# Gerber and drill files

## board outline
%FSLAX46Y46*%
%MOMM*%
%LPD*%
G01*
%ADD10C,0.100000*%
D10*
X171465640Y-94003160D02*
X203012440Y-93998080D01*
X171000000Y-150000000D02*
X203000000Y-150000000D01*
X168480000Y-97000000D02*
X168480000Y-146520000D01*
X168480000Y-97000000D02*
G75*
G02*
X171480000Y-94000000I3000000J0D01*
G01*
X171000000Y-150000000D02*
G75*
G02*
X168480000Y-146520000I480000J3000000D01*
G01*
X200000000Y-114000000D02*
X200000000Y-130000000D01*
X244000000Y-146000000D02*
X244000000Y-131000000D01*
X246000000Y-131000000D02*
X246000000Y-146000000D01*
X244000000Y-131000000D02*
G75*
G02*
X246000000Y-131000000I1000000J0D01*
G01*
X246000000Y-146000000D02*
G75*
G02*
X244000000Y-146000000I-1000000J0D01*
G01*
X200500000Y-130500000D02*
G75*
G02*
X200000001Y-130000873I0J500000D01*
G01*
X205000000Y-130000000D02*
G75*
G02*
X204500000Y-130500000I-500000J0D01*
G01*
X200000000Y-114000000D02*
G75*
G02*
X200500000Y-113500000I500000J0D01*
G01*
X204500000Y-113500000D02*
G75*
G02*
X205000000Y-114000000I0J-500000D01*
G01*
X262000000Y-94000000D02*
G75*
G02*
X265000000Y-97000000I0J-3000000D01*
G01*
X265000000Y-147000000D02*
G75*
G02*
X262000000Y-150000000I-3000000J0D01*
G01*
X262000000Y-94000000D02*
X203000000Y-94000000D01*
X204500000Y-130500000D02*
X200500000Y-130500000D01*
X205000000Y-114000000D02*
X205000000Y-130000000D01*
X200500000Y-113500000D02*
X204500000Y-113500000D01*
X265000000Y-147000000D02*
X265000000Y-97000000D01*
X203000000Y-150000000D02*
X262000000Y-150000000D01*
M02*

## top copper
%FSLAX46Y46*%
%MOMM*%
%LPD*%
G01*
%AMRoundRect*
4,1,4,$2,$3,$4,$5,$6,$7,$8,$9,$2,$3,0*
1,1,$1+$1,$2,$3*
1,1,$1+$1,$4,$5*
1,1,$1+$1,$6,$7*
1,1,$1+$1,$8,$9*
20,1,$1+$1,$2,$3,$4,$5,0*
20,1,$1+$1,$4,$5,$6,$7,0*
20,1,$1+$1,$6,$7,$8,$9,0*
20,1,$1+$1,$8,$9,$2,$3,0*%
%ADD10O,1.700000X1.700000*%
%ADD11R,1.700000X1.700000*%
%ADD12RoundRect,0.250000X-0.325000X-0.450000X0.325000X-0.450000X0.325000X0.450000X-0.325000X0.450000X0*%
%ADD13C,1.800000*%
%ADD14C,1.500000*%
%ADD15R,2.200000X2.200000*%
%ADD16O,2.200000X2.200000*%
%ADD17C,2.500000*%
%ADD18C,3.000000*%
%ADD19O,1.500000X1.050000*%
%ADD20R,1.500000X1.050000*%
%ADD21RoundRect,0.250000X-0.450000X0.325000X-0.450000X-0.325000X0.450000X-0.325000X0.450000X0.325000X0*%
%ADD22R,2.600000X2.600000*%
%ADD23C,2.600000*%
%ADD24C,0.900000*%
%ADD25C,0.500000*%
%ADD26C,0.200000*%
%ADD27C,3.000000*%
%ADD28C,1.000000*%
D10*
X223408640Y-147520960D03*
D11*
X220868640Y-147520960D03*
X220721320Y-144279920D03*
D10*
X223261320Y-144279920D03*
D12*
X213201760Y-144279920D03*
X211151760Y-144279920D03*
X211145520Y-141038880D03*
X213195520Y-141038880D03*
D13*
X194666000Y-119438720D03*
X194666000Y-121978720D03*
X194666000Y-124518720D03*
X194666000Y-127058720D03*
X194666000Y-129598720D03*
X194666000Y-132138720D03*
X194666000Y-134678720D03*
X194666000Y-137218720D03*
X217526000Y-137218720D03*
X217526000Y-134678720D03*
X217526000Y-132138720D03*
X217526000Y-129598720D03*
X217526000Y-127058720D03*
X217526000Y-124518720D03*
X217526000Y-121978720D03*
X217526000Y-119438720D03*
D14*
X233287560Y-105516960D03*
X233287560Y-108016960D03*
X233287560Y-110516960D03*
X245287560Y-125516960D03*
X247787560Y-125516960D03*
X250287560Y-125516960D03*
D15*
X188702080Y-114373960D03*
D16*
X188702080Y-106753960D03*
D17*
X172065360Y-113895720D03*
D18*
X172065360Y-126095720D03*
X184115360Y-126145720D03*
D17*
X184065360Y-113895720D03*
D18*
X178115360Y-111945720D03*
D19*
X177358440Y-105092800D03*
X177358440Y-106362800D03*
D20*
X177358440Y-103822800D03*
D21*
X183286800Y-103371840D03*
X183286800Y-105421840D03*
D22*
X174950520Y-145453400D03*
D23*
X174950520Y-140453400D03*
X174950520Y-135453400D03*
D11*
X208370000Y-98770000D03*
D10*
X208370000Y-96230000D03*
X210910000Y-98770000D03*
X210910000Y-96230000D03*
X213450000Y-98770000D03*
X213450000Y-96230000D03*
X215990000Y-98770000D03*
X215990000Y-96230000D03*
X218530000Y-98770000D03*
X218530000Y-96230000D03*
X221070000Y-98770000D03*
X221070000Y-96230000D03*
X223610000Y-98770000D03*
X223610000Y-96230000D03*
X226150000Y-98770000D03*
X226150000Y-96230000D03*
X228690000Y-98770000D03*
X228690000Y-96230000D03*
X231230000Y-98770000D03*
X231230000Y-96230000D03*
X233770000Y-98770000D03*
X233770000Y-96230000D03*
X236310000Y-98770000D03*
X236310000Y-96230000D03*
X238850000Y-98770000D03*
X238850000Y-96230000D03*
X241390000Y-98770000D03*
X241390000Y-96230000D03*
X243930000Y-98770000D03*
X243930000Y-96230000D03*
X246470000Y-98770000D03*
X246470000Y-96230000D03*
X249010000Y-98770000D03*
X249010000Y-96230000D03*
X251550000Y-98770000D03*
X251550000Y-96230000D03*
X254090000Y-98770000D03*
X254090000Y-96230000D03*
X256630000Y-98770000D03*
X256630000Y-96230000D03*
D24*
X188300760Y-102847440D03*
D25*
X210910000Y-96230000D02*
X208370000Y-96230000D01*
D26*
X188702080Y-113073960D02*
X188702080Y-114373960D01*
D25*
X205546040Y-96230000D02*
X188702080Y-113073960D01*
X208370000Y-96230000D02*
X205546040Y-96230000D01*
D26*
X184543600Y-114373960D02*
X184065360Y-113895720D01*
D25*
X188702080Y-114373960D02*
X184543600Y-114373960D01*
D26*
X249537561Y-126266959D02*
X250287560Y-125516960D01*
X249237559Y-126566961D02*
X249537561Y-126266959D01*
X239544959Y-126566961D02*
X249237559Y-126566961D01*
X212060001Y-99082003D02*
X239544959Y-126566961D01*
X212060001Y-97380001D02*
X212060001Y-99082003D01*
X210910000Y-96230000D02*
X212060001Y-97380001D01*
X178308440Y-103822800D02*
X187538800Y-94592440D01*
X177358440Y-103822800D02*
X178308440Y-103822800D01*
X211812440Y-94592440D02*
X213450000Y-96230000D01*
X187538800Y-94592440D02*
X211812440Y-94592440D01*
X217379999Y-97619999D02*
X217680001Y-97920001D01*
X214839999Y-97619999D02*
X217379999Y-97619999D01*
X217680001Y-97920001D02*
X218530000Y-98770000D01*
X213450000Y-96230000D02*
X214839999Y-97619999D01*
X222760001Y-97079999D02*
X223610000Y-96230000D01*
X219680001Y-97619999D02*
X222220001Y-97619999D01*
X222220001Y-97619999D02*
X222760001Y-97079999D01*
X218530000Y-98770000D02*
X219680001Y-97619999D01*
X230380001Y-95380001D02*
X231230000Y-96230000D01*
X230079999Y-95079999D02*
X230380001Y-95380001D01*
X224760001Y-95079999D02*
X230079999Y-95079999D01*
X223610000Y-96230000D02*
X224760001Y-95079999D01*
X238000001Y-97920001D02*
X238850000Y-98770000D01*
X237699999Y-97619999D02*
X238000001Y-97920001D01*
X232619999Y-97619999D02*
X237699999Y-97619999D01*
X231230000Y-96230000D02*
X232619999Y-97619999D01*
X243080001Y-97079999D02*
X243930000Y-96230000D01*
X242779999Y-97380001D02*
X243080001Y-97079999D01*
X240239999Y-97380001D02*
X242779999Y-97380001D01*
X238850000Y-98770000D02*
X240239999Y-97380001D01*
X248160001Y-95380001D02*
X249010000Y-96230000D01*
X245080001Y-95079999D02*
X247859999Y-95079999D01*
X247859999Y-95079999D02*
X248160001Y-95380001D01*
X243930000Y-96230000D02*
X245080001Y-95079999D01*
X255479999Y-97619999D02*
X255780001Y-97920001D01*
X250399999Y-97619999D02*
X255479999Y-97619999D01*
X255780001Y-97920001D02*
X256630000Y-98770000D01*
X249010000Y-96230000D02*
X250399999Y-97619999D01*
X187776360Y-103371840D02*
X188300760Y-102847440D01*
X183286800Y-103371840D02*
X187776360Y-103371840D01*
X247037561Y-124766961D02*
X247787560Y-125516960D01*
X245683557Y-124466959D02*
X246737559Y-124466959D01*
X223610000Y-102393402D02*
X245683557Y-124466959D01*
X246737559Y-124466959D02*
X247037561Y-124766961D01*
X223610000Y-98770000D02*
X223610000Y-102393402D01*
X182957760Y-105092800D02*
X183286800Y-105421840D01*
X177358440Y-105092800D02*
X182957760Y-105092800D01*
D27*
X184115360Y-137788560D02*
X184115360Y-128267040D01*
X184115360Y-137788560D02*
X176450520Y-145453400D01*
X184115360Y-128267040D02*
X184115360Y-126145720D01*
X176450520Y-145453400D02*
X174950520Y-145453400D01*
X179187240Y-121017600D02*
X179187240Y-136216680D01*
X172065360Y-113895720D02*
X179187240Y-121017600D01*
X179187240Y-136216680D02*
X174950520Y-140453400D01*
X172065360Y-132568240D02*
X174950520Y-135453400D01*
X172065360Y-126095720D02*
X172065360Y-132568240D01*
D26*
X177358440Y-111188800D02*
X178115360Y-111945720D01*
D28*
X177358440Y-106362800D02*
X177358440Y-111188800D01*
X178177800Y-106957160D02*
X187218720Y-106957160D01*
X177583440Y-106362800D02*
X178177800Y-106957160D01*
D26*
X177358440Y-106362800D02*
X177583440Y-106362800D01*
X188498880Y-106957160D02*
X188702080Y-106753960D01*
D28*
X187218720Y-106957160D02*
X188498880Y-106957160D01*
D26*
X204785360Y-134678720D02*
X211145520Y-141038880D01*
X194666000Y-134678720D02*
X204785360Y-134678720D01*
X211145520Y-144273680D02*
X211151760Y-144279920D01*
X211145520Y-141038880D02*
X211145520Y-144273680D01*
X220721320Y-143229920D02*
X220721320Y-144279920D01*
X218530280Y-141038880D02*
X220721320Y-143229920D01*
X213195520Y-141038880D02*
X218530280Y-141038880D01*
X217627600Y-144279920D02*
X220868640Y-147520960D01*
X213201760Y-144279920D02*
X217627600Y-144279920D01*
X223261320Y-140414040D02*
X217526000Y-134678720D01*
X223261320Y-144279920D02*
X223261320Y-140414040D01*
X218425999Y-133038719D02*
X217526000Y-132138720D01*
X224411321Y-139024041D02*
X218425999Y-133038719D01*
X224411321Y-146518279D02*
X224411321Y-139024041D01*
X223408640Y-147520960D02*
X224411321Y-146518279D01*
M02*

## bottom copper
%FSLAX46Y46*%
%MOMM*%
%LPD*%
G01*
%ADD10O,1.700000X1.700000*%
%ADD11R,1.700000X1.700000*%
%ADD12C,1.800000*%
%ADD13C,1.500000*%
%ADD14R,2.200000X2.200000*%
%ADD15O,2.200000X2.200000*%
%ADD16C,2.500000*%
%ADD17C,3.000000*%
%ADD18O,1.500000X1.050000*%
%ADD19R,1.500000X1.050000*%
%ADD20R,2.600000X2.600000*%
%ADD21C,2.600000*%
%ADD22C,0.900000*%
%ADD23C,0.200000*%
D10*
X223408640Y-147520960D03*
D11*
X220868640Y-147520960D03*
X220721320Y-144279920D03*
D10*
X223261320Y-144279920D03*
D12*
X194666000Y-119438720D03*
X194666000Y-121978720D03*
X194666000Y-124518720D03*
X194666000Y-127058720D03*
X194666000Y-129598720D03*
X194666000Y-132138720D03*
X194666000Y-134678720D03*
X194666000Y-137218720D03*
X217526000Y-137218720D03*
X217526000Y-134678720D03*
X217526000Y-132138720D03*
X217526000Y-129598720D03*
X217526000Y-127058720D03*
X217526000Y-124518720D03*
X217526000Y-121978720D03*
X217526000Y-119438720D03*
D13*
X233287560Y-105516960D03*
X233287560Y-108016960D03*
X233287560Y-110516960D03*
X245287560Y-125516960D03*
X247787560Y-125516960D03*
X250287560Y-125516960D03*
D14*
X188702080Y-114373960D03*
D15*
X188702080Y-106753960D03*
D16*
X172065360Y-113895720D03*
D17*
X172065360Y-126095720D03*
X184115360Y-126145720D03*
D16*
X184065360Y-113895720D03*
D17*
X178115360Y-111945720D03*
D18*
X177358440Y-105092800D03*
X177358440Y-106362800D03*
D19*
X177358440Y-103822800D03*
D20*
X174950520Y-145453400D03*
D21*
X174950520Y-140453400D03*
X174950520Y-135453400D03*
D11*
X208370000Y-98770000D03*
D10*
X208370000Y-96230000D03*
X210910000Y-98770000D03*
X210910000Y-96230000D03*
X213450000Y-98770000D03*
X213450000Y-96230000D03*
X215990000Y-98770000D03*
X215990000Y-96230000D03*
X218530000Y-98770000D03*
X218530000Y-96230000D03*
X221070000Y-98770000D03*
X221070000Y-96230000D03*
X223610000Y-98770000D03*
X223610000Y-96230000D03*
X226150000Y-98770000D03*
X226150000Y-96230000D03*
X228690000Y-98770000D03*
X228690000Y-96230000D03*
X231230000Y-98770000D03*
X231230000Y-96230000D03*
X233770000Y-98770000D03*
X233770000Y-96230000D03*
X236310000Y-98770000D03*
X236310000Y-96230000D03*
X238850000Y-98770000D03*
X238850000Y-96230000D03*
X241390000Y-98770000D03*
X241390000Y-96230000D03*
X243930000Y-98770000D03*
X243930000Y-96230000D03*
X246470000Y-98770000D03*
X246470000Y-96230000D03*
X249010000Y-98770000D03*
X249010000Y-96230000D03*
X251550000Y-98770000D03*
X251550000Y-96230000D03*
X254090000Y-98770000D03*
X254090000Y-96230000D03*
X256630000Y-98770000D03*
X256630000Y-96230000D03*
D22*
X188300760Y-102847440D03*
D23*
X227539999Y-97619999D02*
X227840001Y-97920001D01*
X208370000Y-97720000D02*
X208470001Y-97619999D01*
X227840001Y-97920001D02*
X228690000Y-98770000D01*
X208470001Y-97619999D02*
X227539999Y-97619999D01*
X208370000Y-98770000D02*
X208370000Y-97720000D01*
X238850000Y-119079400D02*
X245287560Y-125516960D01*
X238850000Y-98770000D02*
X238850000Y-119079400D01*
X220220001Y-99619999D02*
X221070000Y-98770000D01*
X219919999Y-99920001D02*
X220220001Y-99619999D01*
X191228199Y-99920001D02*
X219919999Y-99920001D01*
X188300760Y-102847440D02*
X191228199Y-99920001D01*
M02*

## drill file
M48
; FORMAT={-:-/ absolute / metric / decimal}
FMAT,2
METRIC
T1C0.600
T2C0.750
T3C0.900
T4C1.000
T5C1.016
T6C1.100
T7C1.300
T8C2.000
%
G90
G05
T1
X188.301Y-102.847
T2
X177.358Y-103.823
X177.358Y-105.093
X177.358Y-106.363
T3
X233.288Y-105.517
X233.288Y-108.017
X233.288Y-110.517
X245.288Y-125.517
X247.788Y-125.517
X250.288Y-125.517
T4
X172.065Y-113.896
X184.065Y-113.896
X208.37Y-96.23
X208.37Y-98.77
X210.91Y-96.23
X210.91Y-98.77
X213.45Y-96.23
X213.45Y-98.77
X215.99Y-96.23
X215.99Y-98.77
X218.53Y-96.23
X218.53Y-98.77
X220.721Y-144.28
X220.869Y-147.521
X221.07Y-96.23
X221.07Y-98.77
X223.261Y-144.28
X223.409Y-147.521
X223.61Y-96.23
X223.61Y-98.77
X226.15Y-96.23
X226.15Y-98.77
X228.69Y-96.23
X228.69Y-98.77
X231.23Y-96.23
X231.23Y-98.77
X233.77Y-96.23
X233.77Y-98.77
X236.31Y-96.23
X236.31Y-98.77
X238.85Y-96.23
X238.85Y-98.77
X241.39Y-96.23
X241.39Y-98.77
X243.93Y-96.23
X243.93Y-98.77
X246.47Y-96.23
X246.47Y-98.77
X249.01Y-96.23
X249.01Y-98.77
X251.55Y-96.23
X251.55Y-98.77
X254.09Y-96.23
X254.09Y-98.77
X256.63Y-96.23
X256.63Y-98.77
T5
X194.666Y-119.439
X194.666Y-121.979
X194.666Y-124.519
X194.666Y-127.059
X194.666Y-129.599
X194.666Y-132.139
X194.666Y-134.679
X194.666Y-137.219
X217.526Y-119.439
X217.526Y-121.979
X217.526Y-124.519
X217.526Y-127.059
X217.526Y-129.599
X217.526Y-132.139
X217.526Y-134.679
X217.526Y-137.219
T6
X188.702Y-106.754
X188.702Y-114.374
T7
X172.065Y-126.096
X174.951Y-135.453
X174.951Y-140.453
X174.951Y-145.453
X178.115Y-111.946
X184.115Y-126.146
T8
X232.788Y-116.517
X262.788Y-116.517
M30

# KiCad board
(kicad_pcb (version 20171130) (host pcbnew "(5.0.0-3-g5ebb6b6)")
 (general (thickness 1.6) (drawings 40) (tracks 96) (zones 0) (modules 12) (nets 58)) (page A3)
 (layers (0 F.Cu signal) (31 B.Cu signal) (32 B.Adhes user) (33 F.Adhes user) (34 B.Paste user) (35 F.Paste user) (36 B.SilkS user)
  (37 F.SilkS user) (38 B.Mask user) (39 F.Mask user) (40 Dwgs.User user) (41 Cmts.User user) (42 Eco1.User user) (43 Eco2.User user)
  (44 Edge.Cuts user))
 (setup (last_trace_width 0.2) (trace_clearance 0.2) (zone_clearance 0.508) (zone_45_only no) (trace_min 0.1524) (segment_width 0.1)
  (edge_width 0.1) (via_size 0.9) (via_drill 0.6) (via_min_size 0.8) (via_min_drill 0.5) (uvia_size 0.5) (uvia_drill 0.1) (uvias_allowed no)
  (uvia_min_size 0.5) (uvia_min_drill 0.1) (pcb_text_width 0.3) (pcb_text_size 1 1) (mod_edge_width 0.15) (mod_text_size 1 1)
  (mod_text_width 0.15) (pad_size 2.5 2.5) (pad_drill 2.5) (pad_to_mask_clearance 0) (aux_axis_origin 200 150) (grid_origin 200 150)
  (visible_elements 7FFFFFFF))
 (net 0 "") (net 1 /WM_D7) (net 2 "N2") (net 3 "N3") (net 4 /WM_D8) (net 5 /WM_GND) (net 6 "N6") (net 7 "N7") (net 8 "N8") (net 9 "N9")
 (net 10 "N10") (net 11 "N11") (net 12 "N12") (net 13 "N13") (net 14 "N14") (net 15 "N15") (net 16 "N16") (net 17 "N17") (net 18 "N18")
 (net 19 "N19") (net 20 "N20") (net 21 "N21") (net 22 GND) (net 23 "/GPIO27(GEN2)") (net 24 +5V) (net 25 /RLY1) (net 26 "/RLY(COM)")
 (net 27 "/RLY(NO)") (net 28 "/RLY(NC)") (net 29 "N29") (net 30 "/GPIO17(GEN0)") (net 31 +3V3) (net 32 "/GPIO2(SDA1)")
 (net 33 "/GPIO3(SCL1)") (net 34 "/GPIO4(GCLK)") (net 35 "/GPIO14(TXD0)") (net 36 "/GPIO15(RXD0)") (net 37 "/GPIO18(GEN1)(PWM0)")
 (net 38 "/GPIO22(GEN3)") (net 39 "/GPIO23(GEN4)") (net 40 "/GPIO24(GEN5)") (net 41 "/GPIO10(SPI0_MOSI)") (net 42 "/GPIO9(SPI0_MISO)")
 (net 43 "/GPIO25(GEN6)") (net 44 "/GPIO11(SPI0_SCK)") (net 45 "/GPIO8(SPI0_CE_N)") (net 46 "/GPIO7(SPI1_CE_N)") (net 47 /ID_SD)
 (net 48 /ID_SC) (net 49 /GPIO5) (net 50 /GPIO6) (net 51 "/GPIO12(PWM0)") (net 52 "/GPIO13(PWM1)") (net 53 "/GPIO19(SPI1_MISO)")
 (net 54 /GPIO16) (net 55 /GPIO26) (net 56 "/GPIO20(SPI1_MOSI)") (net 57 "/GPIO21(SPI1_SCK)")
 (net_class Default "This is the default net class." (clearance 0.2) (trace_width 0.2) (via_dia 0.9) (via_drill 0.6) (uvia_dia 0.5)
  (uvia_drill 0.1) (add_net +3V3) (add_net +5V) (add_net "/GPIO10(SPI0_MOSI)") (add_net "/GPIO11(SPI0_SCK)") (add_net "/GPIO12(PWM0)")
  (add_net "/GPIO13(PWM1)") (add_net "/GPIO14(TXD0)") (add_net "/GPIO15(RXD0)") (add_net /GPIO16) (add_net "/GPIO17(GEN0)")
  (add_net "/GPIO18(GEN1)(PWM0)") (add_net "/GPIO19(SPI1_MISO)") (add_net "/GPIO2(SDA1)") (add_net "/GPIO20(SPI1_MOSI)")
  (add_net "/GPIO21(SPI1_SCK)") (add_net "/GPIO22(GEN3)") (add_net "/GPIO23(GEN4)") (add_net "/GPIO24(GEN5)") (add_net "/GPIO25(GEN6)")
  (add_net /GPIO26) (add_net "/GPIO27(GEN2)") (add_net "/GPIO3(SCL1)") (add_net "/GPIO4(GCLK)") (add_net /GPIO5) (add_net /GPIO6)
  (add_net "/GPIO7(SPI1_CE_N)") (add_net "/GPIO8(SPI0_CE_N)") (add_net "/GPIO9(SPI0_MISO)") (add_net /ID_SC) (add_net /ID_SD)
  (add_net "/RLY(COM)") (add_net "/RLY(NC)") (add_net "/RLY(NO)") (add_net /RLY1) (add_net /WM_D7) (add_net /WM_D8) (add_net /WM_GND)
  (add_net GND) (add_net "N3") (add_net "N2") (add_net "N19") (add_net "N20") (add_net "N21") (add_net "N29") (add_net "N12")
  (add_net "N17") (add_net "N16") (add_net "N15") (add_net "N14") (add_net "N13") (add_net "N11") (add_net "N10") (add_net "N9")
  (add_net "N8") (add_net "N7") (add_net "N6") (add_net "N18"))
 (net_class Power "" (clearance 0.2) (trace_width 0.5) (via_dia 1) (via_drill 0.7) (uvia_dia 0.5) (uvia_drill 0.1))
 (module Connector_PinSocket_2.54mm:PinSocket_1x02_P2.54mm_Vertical (layer F.Cu) (at 220.86864 147.52096 90)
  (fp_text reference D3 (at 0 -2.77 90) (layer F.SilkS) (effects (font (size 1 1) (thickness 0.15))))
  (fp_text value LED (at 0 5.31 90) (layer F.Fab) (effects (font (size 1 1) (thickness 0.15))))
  (pad 2 thru_hole oval (at 0 2.54 90) (size 1.7 1.7) (drill 1) (layers *.Cu *.Mask) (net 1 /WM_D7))
  (pad 1 thru_hole rect (at 0 0 90) (size 1.7 1.7) (drill 1) (layers *.Cu *.Mask) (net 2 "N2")))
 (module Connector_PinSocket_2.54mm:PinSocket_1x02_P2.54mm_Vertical (layer F.Cu) (at 220.72132 144.27992 90)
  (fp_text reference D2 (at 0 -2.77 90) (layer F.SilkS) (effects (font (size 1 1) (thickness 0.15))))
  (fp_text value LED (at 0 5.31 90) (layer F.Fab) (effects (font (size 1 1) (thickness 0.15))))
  (pad 1 thru_hole rect (at 0 0 90) (size 1.7 1.7) (drill 1) (layers *.Cu *.Mask) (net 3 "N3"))
  (pad 2 thru_hole oval (at 0 2.54 90) (size 1.7 1.7) (drill 1) (layers *.Cu *.Mask) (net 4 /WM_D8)))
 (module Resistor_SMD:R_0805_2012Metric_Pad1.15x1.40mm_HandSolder (layer F.Cu) (at 212.17676 144.27992)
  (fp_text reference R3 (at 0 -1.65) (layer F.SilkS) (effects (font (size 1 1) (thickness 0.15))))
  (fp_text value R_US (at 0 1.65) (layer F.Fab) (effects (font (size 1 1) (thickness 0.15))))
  (pad 2 smd roundrect (at 1.025 0) (size 1.15 1.4) (layers F.Cu F.Paste F.Mask) (roundrect_rratio 0.217391) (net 2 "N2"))
  (pad 1 smd roundrect (at -1.025 0) (size 1.15 1.4) (layers F.Cu F.Paste F.Mask) (roundrect_rratio 0.217391) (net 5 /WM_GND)))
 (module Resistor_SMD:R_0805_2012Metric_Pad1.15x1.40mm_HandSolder (layer F.Cu) (at 212.17052 141.03888)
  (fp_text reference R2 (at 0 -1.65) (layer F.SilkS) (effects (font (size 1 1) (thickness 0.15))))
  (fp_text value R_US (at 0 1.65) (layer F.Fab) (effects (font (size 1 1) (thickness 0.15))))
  (pad 1 smd roundrect (at -1.025 0) (size 1.15 1.4) (layers F.Cu F.Paste F.Mask) (roundrect_rratio 0.217391) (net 5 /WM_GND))
  (pad 2 smd roundrect (at 1.025 0) (size 1.15 1.4) (layers F.Cu F.Paste F.Mask) (roundrect_rratio 0.217391) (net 3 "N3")))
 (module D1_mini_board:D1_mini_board (layer F.Cu) (at 206.096 129.59872)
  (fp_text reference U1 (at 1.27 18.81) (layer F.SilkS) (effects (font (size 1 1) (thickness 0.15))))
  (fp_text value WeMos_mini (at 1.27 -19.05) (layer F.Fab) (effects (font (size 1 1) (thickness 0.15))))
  (pad 8 thru_hole circle (at -11.43 -10.16) (size 1.8 1.8) (drill 1.016) (layers *.Cu *.Mask F.SilkS) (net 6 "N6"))
  (pad 7 thru_hole circle (at -11.43 -7.62) (size 1.8 1.8) (drill 1.016) (layers *.Cu *.Mask F.SilkS) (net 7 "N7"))
  (pad 6 thru_hole circle (at -11.43 -5.08) (size 1.8 1.8) (drill 1.016) (layers *.Cu *.Mask F.SilkS) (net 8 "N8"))
  (pad 5 thru_hole circle (at -11.43 -2.54) (size 1.8 1.8) (drill 1.016) (layers *.Cu *.Mask F.SilkS) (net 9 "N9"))
  (pad 4 thru_hole circle (at -11.43 0) (size 1.8 1.8) (drill 1.016) (layers *.Cu *.Mask F.SilkS) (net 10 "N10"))
  (pad 3 thru_hole circle (at -11.43 2.54) (size 1.8 1.8) (drill 1.016) (layers *.Cu *.Mask F.SilkS) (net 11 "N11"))
  (pad 2 thru_hole circle (at -11.43 5.08) (size 1.8 1.8) (drill 1.016) (layers *.Cu *.Mask F.SilkS) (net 5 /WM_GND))
  (pad 1 thru_hole circle (at -11.43 7.62) (size 1.8 1.8) (drill 1.016) (layers *.Cu *.Mask F.SilkS) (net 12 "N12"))
  (pad 16 thru_hole circle (at 11.43 7.62) (size 1.8 1.8) (drill 1.016) (layers *.Cu *.Mask F.SilkS) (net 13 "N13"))
  (pad 15 thru_hole circle (at 11.43 5.08) (size 1.8 1.8) (drill 1.016) (layers *.Cu *.Mask F.SilkS) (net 4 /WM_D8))
  (pad 14 thru_hole circle (at 11.43 2.54) (size 1.8 1.8) (drill 1.016) (layers *.Cu *.Mask F.SilkS) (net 1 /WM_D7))
  (pad 13 thru_hole circle (at 11.43 0) (size 1.8 1.8) (drill 1.016) (layers *.Cu *.Mask F.SilkS) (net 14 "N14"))
  (pad 12 thru_hole circle (at 11.43 -2.54) (size 1.8 1.8) (drill 1.016) (layers *.Cu *.Mask F.SilkS) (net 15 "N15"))
  (pad 11 thru_hole circle (at 11.43 -5.08) (size 1.8 1.8) (drill 1.016) (layers *.Cu *.Mask F.SilkS) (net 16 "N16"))
  (pad 10 thru_hole circle (at 11.43 -7.62) (size 1.8 1.8) (drill 1.016) (layers *.Cu *.Mask F.SilkS) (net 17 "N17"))
  (pad 9 thru_hole circle (at 11.43 -10.16) (size 1.8 1.8) (drill 1.016) (layers *.Cu *.Mask F.SilkS) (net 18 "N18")))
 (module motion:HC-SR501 (layer F.Cu) (at 247.78756 115.51696)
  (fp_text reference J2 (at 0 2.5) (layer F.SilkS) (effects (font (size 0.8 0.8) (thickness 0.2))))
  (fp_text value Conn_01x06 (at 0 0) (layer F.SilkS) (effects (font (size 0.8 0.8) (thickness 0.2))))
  (pad 1 thru_hole circle (at -14.5 -10) (size 1.5 1.5) (drill 0.9) (layers *.Cu *.Mask F.SilkS) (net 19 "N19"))
  (pad 2 thru_hole circle (at -14.5 -7.5) (size 1.5 1.5) (drill 0.9) (layers *.Cu *.Mask F.SilkS) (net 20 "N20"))
  (pad 3 thru_hole circle (at -14.5 -5) (size 1.5 1.5) (drill 0.9) (layers *.Cu *.Mask F.SilkS) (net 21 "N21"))
  (pad 4 thru_hole circle (at -2.5 10) (size 1.5 1.5) (drill 0.9) (layers *.Cu *.Mask F.SilkS) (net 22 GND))
  (pad 5 thru_hole circle (at 0 10) (size 1.5 1.5) (drill 0.9) (layers *.Cu *.Mask F.SilkS) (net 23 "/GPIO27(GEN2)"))
  (pad 6 thru_hole circle (at 2.5 10) (size 1.5 1.5) (drill 0.9) (layers *.Cu *.Mask F.SilkS) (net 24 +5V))
  (pad "" np_thru_hole circle (at 15 1) (size 2 2) (drill 2) (layers *.Cu *.Mask F.SilkS))
  (pad "" np_thru_hole circle (at -15 1) (size 2 2) (drill 2) (layers *.Cu *.Mask F.SilkS)))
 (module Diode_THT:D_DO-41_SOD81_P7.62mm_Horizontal (layer F.Cu) (at 188.70208 114.37396 90)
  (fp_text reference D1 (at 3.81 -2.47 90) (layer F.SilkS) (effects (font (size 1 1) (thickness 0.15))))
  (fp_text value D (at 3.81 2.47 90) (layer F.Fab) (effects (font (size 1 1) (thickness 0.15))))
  (pad 1 thru_hole rect (at 0 0 90) (size 2.2 2.2) (drill 1.1) (layers *.Cu *.Mask) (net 24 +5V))
  (pad 2 thru_hole oval (at 7.62 0 90) (size 2.2 2.2) (drill 1.1) (layers *.Cu *.Mask) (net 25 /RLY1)))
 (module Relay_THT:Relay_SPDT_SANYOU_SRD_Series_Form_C (layer F.Cu) (at 178.11536 111.94572 270)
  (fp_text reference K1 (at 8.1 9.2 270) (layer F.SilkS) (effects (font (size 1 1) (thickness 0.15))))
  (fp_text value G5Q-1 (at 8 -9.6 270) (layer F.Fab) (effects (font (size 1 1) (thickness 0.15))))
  (pad 2 thru_hole circle (at 1.95 6.05) (size 2.5 2.5) (drill 1) (layers *.Cu *.Mask) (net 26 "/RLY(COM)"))
  (pad 3 thru_hole circle (at 14.15 6.05) (size 3 3) (drill 1.3) (layers *.Cu *.Mask) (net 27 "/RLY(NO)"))
  (pad 4 thru_hole circle (at 14.2 -6) (size 3 3) (drill 1.3) (layers *.Cu *.Mask) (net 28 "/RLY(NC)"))
  (pad 5 thru_hole circle (at 1.95 -5.95) (size 2.5 2.5) (drill 1) (layers *.Cu *.Mask) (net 24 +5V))
  (pad 1 thru_hole circle (at 0 0) (size 3 3) (drill 1.3) (layers *.Cu *.Mask) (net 25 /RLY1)))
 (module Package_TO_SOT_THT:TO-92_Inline (layer F.Cu) (at 177.35844 103.8228 270)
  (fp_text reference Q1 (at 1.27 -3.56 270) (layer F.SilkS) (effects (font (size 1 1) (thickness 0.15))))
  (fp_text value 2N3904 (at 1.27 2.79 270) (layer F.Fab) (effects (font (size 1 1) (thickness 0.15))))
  (pad 2 thru_hole oval (at 1.27 0 270) (size 1.05 1.5) (drill 0.75) (layers *.Cu *.Mask) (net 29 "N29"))
  (pad 3 thru_hole oval (at 2.54 0 270) (size 1.05 1.5) (drill 0.75) (layers *.Cu *.Mask) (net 25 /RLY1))
  (pad 1 thru_hole rect (at 0 0 270) (size 1.05 1.5) (drill 0.75) (layers *.Cu *.Mask) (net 22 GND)))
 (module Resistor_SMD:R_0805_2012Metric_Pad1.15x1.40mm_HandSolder (layer F.Cu) (at 183.2868 104.39684 270)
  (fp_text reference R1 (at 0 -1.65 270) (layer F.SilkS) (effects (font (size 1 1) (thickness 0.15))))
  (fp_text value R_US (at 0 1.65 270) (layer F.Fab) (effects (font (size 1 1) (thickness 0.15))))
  (pad 1 smd roundrect (at -1.025 0 270) (size 1.15 1.4) (layers F.Cu F.Paste F.Mask) (roundrect_rratio 0.217391) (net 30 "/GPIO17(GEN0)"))
  (pad 2 smd roundrect (at 1.025 0 270) (size 1.15 1.4) (layers F.Cu F.Paste F.Mask) (roundrect_rratio 0.217391) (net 29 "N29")))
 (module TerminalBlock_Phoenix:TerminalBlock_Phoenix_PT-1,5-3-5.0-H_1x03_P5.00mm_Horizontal (layer F.Cu) (at 174.95052 145.4534 90)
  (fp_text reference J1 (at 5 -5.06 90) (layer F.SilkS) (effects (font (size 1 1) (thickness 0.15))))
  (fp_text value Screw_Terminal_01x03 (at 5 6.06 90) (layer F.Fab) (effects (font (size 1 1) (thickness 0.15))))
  (pad 1 thru_hole rect (at 0 0 90) (size 2.6 2.6) (drill 1.3) (layers *.Cu *.Mask) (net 28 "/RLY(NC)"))
  (pad 2 thru_hole circle (at 5 0 90) (size 2.6 2.6) (drill 1.3) (layers *.Cu *.Mask) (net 26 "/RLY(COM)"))
  (pad 3 thru_hole circle (at 10 0 90) (size 2.6 2.6) (drill 1.3) (layers *.Cu *.Mask) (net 27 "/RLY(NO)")))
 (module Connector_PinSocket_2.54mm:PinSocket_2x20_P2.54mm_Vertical (layer B.Cu) (at 208.37 98.77 270)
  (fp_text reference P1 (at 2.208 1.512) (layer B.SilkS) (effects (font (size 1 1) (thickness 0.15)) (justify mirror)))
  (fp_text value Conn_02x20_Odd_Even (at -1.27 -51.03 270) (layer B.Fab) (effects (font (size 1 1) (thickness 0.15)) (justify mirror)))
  (pad 1 thru_hole rect (at 0 0 270) (size 1.7 1.7) (drill 1) (layers *.Cu *.Mask) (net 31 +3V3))
  (pad 2 thru_hole oval (at -2.54 0 270) (size 1.7 1.7) (drill 1) (layers *.Cu *.Mask) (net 24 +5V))
  (pad 3 thru_hole oval (at 0 -2.54 270) (size 1.7 1.7) (drill 1) (layers *.Cu *.Mask) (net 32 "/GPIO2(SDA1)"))
  (pad 4 thru_hole oval (at -2.54 -2.54 270) (size 1.7 1.7) (drill 1) (layers *.Cu *.Mask) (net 24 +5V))
  (pad 5 thru_hole oval (at 0 -5.08 270) (size 1.7 1.7) (drill 1) (layers *.Cu *.Mask) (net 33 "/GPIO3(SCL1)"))
  (pad 6 thru_hole oval (at -2.54 -5.08 270) (size 1.7 1.7) (drill 1) (layers *.Cu *.Mask) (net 22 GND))
  (pad 7 thru_hole oval (at 0 -7.62 270) (size 1.7 1.7) (drill 1) (layers *.Cu *.Mask) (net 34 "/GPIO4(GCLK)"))
  (pad 8 thru_hole oval (at -2.54 -7.62 270) (size 1.7 1.7) (drill 1) (layers *.Cu *.Mask) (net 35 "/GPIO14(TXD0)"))
  (pad 9 thru_hole oval (at 0 -10.16 270) (size 1.7 1.7) (drill 1) (layers *.Cu *.Mask) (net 22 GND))
  (pad 10 thru_hole oval (at -2.54 -10.16 270) (size 1.7 1.7) (drill 1) (layers *.Cu *.Mask) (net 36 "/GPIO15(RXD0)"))
  (pad 11 thru_hole oval (at 0 -12.7 270) (size 1.7 1.7) (drill 1) (layers *.Cu *.Mask) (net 30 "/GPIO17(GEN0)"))
  (pad 12 thru_hole oval (at -2.54 -12.7 270) (size 1.7 1.7) (drill 1) (layers *.Cu *.Mask) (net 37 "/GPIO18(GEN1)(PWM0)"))
  (pad 13 thru_hole oval (at 0 -15.24 270) (size 1.7 1.7) (drill 1) (layers *.Cu *.Mask) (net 23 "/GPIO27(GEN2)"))
  (pad 14 thru_hole oval (at -2.54 -15.24 270) (size 1.7 1.7) (drill 1) (layers *.Cu *.Mask) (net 22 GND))
  (pad 15 thru_hole oval (at 0 -17.78 270) (size 1.7 1.7) (drill 1) (layers *.Cu *.Mask) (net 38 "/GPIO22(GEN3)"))
  (pad 16 thru_hole oval (at -2.54 -17.78 270) (size 1.7 1.7) (drill 1) (layers *.Cu *.Mask) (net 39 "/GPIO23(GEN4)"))
  (pad 17 thru_hole oval (at 0 -20.32 270) (size 1.7 1.7) (drill 1) (layers *.Cu *.Mask) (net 31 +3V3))
  (pad 18 thru_hole oval (at -2.54 -20.32 270) (size 1.7 1.7) (drill 1) (layers *.Cu *.Mask) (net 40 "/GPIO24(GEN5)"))
  (pad 19 thru_hole oval (at 0 -22.86 270) (size 1.7 1.7) (drill 1) (layers *.Cu *.Mask) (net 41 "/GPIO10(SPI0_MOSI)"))
  (pad 20 thru_hole oval (at -2.54 -22.86 270) (size 1.7 1.7) (drill 1) (layers *.Cu *.Mask) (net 22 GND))
  (pad 21 thru_hole oval (at 0 -25.4 270) (size 1.7 1.7) (drill 1) (layers *.Cu *.Mask) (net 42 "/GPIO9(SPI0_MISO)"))
  (pad 22 thru_hole oval (at -2.54 -25.4 270) (size 1.7 1.7) (drill 1) (layers *.Cu *.Mask) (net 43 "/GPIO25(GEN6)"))
  (pad 23 thru_hole oval (at 0 -27.94 270) (size 1.7 1.7) (drill 1) (layers *.Cu *.Mask) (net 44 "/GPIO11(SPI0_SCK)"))
  (pad 24 thru_hole oval (at -2.54 -27.94 270) (size 1.7 1.7) (drill 1) (layers *.Cu *.Mask) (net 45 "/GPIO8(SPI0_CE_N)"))
  (pad 25 thru_hole oval (at 0 -30.48 270) (size 1.7 1.7) (drill 1) (layers *.Cu *.Mask) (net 22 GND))
  (pad 26 thru_hole oval (at -2.54 -30.48 270) (size 1.7 1.7) (drill 1) (layers *.Cu *.Mask) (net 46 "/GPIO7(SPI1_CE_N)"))
  (pad 27 thru_hole oval (at 0 -33.02 270) (size 1.7 1.7) (drill 1) (layers *.Cu *.Mask) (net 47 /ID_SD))
  (pad 28 thru_hole oval (at -2.54 -33.02 270) (size 1.7 1.7) (drill 1) (layers *.Cu *.Mask) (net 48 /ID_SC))
  (pad 29 thru_hole oval (at 0 -35.56 270) (size 1.7 1.7) (drill 1) (layers *.Cu *.Mask) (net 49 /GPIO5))
  (pad 30 thru_hole oval (at -2.54 -35.56 270) (size 1.7 1.7) (drill 1) (layers *.Cu *.Mask) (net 22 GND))
  (pad 31 thru_hole oval (at 0 -38.1 270) (size 1.7 1.7) (drill 1) (layers *.Cu *.Mask) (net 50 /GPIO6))
  (pad 32 thru_hole oval (at -2.54 -38.1 270) (size 1.7 1.7) (drill 1) (layers *.Cu *.Mask) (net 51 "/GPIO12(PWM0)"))
  (pad 33 thru_hole oval (at 0 -40.64 270) (size 1.7 1.7) (drill 1) (layers *.Cu *.Mask) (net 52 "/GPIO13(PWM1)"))
  (pad 34 thru_hole oval (at -2.54 -40.64 270) (size 1.7 1.7) (drill 1) (layers *.Cu *.Mask) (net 22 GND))
  (pad 35 thru_hole oval (at 0 -43.18 270) (size 1.7 1.7) (drill 1) (layers *.Cu *.Mask) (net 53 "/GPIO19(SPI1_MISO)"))
  (pad 36 thru_hole oval (at -2.54 -43.18 270) (size 1.7 1.7) (drill 1) (layers *.Cu *.Mask) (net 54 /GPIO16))
  (pad 37 thru_hole oval (at 0 -45.72 270) (size 1.7 1.7) (drill 1) (layers *.Cu *.Mask) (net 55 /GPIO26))
  (pad 38 thru_hole oval (at -2.54 -45.72 270) (size 1.7 1.7) (drill 1) (layers *.Cu *.Mask) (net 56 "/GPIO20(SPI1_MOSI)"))
  (pad 39 thru_hole oval (at 0 -48.26 270) (size 1.7 1.7) (drill 1) (layers *.Cu *.Mask) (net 22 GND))
  (pad 40 thru_hole oval (at -2.54 -48.26 270) (size 1.7 1.7) (drill 1) (layers *.Cu *.Mask) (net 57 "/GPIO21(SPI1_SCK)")))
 (gr_line (start 171.46564 94.00316) (end 203.01244 93.99808) (layer Edge.Cuts) (width 0.1))
 (gr_line (start 171 150) (end 203 150) (layer Edge.Cuts) (width 0.1))
 (gr_line (start 168.48 97) (end 168.48 146.52) (layer Edge.Cuts) (width 0.1))
 (gr_arc (start 171.48 97) (end 168.48 97) (angle 90) (layer Edge.Cuts) (width 0.1))
 (gr_arc (start 171.48 147) (end 171 150) (angle 90) (layer Edge.Cuts) (width 0.1))
 (gr_line (start 200 114) (end 200 130) (layer Edge.Cuts) (width 0.1))
 (gr_line (start 244 146) (end 244 131) (layer Edge.Cuts) (width 0.1))
 (gr_line (start 246 131) (end 246 146) (layer Edge.Cuts) (width 0.1))
 (gr_arc (start 245 131) (end 244 131) (angle 180) (layer Edge.Cuts) (width 0.1))
 (gr_arc (start 245 146) (end 246 146) (angle 180) (layer Edge.Cuts) (width 0.1))
 (gr_arc (start 200.5 130) (end 200.5 130.5) (angle 89.89996147) (layer Edge.Cuts) (width 0.1))
 (gr_arc (start 204.5 130) (end 205 130) (angle 90) (layer Edge.Cuts) (width 0.1))
 (gr_arc (start 200.5 114) (end 200 114) (angle 90) (layer Edge.Cuts) (width 0.1))
 (gr_arc (start 204.5 114) (end 204.5 113.5) (angle 90) (layer Edge.Cuts) (width 0.1))
 (gr_arc (start 262 97) (end 262 94) (angle 90) (layer Edge.Cuts) (width 0.1))
 (gr_arc (start 262 147) (end 265 147) (angle 90) (layer Edge.Cuts) (width 0.1))
 (gr_line (start 262 94) (end 203 94) (layer Edge.Cuts) (width 0.1))
 (gr_line (start 204.5 130.5) (end 200.5 130.5) (layer Edge.Cuts) (width 0.1))
 (gr_line (start 205 114) (end 205 130) (layer Edge.Cuts) (width 0.1))
 (gr_line (start 200.5 113.5) (end 204.5 113.5) (layer Edge.Cuts) (width 0.1))
 (gr_line (start 265 147) (end 265 97) (layer Edge.Cuts) (width 0.1))
 (gr_line (start 203 150) (end 262 150) (layer Edge.Cuts) (width 0.1))
 (segment (start 227.539999 97.619999) (end 227.840001 97.920001) (width 0.2) (layer B.Cu) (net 31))
 (segment (start 208.37 97.72) (end 208.470001 97.619999) (width 0.2) (layer B.Cu) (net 31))
 (segment (start 227.840001 97.920001) (end 228.69 98.77) (width 0.2) (layer B.Cu) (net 31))
 (segment (start 208.470001 97.619999) (end 227.539999 97.619999) (width 0.2) (layer B.Cu) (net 31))
 (segment (start 208.37 98.77) (end 208.37 97.72) (width 0.2) (layer B.Cu) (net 31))
 (segment (start 210.91 96.23) (end 208.37 96.23) (width 0.5) (layer F.Cu) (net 24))
 (segment (start 188.70208 113.07396) (end 188.70208 114.37396) (width 0.2) (layer F.Cu) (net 24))
 (segment (start 205.54604 96.23) (end 188.70208 113.07396) (width 0.5) (layer F.Cu) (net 24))
 (segment (start 208.37 96.23) (end 205.54604 96.23) (width 0.5) (layer F.Cu) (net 24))
 (segment (start 184.5436 114.37396) (end 184.06536 113.89572) (width 0.2) (layer F.Cu) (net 24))
 (segment (start 188.70208 114.37396) (end 184.5436 114.37396) (width 0.5) (layer F.Cu) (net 24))
 (segment (start 249.537561 126.266959) (end 250.28756 125.51696) (width 0.2) (layer F.Cu) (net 24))
 (segment (start 249.237559 126.566961) (end 249.537561 126.266959) (width 0.2) (layer F.Cu) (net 24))
 (segment (start 239.544959 126.566961) (end 249.237559 126.566961) (width 0.2) (layer F.Cu) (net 24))
 (segment (start 212.060001 99.082003) (end 239.544959 126.566961) (width 0.2) (layer F.Cu) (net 24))
 (segment (start 212.060001 97.380001) (end 212.060001 99.082003) (width 0.2) (layer F.Cu) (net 24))
 (segment (start 210.91 96.23) (end 212.060001 97.380001) (width 0.2) (layer F.Cu) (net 24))
 (segment (start 178.30844 103.8228) (end 187.5388 94.59244) (width 0.2) (layer F.Cu) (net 22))
 (segment (start 177.35844 103.8228) (end 178.30844 103.8228) (width 0.2) (layer F.Cu) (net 22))
 (segment (start 211.81244 94.59244) (end 213.45 96.23) (width 0.2) (layer F.Cu) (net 22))
 (segment (start 187.5388 94.59244) (end 211.81244 94.59244) (width 0.2) (layer F.Cu) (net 22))
 (segment (start 217.379999 97.619999) (end 217.680001 97.920001) (width 0.2) (layer F.Cu) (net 22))
 (segment (start 214.839999 97.619999) (end 217.379999 97.619999) (width 0.2) (layer F.Cu) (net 22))
 (segment (start 217.680001 97.920001) (end 218.53 98.77) (width 0.2) (layer F.Cu) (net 22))
 (segment (start 213.45 96.23) (end 214.839999 97.619999) (width 0.2) (layer F.Cu) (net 22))
 (segment (start 222.760001 97.079999) (end 223.61 96.23) (width 0.2) (layer F.Cu) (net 22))
 (segment (start 219.680001 97.619999) (end 222.220001 97.619999) (width 0.2) (layer F.Cu) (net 22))
 (segment (start 222.220001 97.619999) (end 222.760001 97.079999) (width 0.2) (layer F.Cu) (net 22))
 (segment (start 218.53 98.77) (end 219.680001 97.619999) (width 0.2) (layer F.Cu) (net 22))
 (segment (start 230.380001 95.380001) (end 231.23 96.23) (width 0.2) (layer F.Cu) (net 22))
 (segment (start 230.079999 95.079999) (end 230.380001 95.380001) (width 0.2) (layer F.Cu) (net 22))
 (segment (start 224.760001 95.079999) (end 230.079999 95.079999) (width 0.2) (layer F.Cu) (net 22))
 (segment (start 223.61 96.23) (end 224.760001 95.079999) (width 0.2) (layer F.Cu) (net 22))
 (segment (start 238.000001 97.920001) (end 238.85 98.77) (width 0.2) (layer F.Cu) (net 22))
 (segment (start 237.699999 97.619999) (end 238.000001 97.920001) (width 0.2) (layer F.Cu) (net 22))
 (segment (start 232.619999 97.619999) (end 237.699999 97.619999) (width 0.2) (layer F.Cu) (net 22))
 (segment (start 231.23 96.23) (end 232.619999 97.619999) (width 0.2) (layer F.Cu) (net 22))
 (segment (start 243.080001 97.079999) (end 243.93 96.23) (width 0.2) (layer F.Cu) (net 22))
 (segment (start 242.779999 97.380001) (end 243.080001 97.079999) (width 0.2) (layer F.Cu) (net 22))
 (segment (start 240.239999 97.380001) (end 242.779999 97.380001) (width 0.2) (layer F.Cu) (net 22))
 (segment (start 238.85 98.77) (end 240.239999 97.380001) (width 0.2) (layer F.Cu) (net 22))
 (segment (start 248.160001 95.380001) (end 249.01 96.23) (width 0.2) (layer F.Cu) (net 22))
 (segment (start 245.080001 95.079999) (end 247.859999 95.079999) (width 0.2) (layer F.Cu) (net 22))
 (segment (start 247.859999 95.079999) (end 248.160001 95.380001) (width 0.2) (layer F.Cu) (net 22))
 (segment (start 243.93 96.23) (end 245.080001 95.079999) (width 0.2) (layer F.Cu) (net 22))
 (segment (start 255.479999 97.619999) (end 255.780001 97.920001) (width 0.2) (layer F.Cu) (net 22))
 (segment (start 250.399999 97.619999) (end 255.479999 97.619999) (width 0.2) (layer F.Cu) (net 22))
 (segment (start 255.780001 97.920001) (end 256.63 98.77) (width 0.2) (layer F.Cu) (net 22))
 (segment (start 249.01 96.23) (end 250.399999 97.619999) (width 0.2) (layer F.Cu) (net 22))
 (segment (start 238.85 119.0794) (end 245.28756 125.51696) (width 0.2) (layer B.Cu) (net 22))
 (segment (start 238.85 98.77) (end 238.85 119.0794) (width 0.2) (layer B.Cu) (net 22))
 (via (at 188.30076 102.84744) (size 0.9) (drill 0.6) (layers F.Cu B.Cu) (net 30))
 (segment (start 187.77636 103.37184) (end 188.30076 102.84744) (width 0.2) (layer F.Cu) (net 30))
 (segment (start 183.2868 103.37184) (end 187.77636 103.37184) (width 0.2) (layer F.Cu) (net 30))
 (segment (start 220.220001 99.619999) (end 221.07 98.77) (width 0.2) (layer B.Cu) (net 30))
 (segment (start 219.919999 99.920001) (end 220.220001 99.619999) (width 0.2) (layer B.Cu) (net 30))
 (segment (start 191.228199 99.920001) (end 219.919999 99.920001) (width 0.2) (layer B.Cu) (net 30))
 (segment (start 188.30076 102.84744) (end 191.228199 99.920001) (width 0.2) (layer B.Cu) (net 30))
 (segment (start 247.037561 124.766961) (end 247.78756 125.51696) (width 0.2) (layer F.Cu) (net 23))
 (segment (start 245.683557 124.466959) (end 246.737559 124.466959) (width 0.2) (layer F.Cu) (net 23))
 (segment (start 223.61 102.393402) (end 245.683557 124.466959) (width 0.2) (layer F.Cu) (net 23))
 (segment (start 246.737559 124.466959) (end 247.037561 124.766961) (width 0.2) (layer F.Cu) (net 23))
 (segment (start 223.61 98.77) (end 223.61 102.393402) (width 0.2) (layer F.Cu) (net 23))
 (segment (start 182.95776 105.0928) (end 183.2868 105.42184) (width 0.2) (layer F.Cu) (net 29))
 (segment (start 177.35844 105.0928) (end 182.95776 105.0928) (width 0.2) (layer F.Cu) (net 29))
 (segment (start 184.11536 137.78856) (end 184.11536 128.26704) (width 3) (layer F.Cu) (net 28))
 (segment (start 184.11536 137.78856) (end 176.45052 145.4534) (width 3) (layer F.Cu) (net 28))
 (segment (start 184.11536 128.26704) (end 184.11536 126.14572) (width 3) (layer F.Cu) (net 28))
 (segment (start 176.45052 145.4534) (end 174.95052 145.4534) (width 3) (layer F.Cu) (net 28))
 (segment (start 179.18724 121.0176) (end 179.18724 136.21668) (width 3) (layer F.Cu) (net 26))
 (segment (start 172.06536 113.89572) (end 179.18724 121.0176) (width 3) (layer F.Cu) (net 26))
 (segment (start 179.18724 136.21668) (end 174.95052 140.4534) (width 3) (layer F.Cu) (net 26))
 (segment (start 172.06536 132.56824) (end 174.95052 135.4534) (width 3) (layer F.Cu) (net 27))
 (segment (start 172.06536 126.09572) (end 172.06536 132.56824) (width 3) (layer F.Cu) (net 27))
 (segment (start 177.35844 111.1888) (end 178.11536 111.94572) (width 0.2) (layer F.Cu) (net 25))
 (segment (start 177.35844 106.3628) (end 177.35844 111.1888) (width 1) (layer F.Cu) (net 25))
 (segment (start 178.1778 106.95716) (end 187.21872 106.95716) (width 1) (layer F.Cu) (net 25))
 (segment (start 177.58344 106.3628) (end 178.1778 106.95716) (width 1) (layer F.Cu) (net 25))
 (segment (start 177.35844 106.3628) (end 177.58344 106.3628) (width 0.2) (layer F.Cu) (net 25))
 (segment (start 188.49888 106.95716) (end 188.70208 106.75396) (width 0.2) (layer F.Cu) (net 25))
 (segment (start 187.21872 106.95716) (end 188.49888 106.95716) (width 1) (layer F.Cu) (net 25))
 (segment (start 204.78536 134.67872) (end 211.14552 141.03888) (width 0.2) (layer F.Cu) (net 5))
 (segment (start 194.666 134.67872) (end 204.78536 134.67872) (width 0.2) (layer F.Cu) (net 5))
 (segment (start 211.14552 144.27368) (end 211.15176 144.27992) (width 0.2) (layer F.Cu) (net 5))
 (segment (start 211.14552 141.03888) (end 211.14552 144.27368) (width 0.2) (layer F.Cu) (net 5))
 (segment (start 220.72132 143.22992) (end 220.72132 144.27992) (width 0.2) (layer F.Cu) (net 3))
 (segment (start 218.53028 141.03888) (end 220.72132 143.22992) (width 0.2) (layer F.Cu) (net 3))
 (segment (start 213.19552 141.03888) (end 218.53028 141.03888) (width 0.2) (layer F.Cu) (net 3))
 (segment (start 217.6276 144.27992) (end 220.86864 147.52096) (width 0.2) (layer F.Cu) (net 2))
 (segment (start 213.20176 144.27992) (end 217.6276 144.27992) (width 0.2) (layer F.Cu) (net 2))
 (segment (start 223.26132 140.41404) (end 217.526 134.67872) (width 0.2) (layer F.Cu) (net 4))
 (segment (start 223.26132 144.27992) (end 223.26132 140.41404) (width 0.2) (layer F.Cu) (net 4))
 (segment (start 218.425999 133.038719) (end 217.526 132.13872) (width 0.2) (layer F.Cu) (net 1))
 (segment (start 224.411321 139.024041) (end 218.425999 133.038719) (width 0.2) (layer F.Cu) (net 1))
 (segment (start 224.411321 146.518279) (end 224.411321 139.024041) (width 0.2) (layer F.Cu) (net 1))
 (segment (start 223.40864 147.52096) (end 224.411321 146.518279) (width 0.2) (layer F.Cu) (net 1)))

